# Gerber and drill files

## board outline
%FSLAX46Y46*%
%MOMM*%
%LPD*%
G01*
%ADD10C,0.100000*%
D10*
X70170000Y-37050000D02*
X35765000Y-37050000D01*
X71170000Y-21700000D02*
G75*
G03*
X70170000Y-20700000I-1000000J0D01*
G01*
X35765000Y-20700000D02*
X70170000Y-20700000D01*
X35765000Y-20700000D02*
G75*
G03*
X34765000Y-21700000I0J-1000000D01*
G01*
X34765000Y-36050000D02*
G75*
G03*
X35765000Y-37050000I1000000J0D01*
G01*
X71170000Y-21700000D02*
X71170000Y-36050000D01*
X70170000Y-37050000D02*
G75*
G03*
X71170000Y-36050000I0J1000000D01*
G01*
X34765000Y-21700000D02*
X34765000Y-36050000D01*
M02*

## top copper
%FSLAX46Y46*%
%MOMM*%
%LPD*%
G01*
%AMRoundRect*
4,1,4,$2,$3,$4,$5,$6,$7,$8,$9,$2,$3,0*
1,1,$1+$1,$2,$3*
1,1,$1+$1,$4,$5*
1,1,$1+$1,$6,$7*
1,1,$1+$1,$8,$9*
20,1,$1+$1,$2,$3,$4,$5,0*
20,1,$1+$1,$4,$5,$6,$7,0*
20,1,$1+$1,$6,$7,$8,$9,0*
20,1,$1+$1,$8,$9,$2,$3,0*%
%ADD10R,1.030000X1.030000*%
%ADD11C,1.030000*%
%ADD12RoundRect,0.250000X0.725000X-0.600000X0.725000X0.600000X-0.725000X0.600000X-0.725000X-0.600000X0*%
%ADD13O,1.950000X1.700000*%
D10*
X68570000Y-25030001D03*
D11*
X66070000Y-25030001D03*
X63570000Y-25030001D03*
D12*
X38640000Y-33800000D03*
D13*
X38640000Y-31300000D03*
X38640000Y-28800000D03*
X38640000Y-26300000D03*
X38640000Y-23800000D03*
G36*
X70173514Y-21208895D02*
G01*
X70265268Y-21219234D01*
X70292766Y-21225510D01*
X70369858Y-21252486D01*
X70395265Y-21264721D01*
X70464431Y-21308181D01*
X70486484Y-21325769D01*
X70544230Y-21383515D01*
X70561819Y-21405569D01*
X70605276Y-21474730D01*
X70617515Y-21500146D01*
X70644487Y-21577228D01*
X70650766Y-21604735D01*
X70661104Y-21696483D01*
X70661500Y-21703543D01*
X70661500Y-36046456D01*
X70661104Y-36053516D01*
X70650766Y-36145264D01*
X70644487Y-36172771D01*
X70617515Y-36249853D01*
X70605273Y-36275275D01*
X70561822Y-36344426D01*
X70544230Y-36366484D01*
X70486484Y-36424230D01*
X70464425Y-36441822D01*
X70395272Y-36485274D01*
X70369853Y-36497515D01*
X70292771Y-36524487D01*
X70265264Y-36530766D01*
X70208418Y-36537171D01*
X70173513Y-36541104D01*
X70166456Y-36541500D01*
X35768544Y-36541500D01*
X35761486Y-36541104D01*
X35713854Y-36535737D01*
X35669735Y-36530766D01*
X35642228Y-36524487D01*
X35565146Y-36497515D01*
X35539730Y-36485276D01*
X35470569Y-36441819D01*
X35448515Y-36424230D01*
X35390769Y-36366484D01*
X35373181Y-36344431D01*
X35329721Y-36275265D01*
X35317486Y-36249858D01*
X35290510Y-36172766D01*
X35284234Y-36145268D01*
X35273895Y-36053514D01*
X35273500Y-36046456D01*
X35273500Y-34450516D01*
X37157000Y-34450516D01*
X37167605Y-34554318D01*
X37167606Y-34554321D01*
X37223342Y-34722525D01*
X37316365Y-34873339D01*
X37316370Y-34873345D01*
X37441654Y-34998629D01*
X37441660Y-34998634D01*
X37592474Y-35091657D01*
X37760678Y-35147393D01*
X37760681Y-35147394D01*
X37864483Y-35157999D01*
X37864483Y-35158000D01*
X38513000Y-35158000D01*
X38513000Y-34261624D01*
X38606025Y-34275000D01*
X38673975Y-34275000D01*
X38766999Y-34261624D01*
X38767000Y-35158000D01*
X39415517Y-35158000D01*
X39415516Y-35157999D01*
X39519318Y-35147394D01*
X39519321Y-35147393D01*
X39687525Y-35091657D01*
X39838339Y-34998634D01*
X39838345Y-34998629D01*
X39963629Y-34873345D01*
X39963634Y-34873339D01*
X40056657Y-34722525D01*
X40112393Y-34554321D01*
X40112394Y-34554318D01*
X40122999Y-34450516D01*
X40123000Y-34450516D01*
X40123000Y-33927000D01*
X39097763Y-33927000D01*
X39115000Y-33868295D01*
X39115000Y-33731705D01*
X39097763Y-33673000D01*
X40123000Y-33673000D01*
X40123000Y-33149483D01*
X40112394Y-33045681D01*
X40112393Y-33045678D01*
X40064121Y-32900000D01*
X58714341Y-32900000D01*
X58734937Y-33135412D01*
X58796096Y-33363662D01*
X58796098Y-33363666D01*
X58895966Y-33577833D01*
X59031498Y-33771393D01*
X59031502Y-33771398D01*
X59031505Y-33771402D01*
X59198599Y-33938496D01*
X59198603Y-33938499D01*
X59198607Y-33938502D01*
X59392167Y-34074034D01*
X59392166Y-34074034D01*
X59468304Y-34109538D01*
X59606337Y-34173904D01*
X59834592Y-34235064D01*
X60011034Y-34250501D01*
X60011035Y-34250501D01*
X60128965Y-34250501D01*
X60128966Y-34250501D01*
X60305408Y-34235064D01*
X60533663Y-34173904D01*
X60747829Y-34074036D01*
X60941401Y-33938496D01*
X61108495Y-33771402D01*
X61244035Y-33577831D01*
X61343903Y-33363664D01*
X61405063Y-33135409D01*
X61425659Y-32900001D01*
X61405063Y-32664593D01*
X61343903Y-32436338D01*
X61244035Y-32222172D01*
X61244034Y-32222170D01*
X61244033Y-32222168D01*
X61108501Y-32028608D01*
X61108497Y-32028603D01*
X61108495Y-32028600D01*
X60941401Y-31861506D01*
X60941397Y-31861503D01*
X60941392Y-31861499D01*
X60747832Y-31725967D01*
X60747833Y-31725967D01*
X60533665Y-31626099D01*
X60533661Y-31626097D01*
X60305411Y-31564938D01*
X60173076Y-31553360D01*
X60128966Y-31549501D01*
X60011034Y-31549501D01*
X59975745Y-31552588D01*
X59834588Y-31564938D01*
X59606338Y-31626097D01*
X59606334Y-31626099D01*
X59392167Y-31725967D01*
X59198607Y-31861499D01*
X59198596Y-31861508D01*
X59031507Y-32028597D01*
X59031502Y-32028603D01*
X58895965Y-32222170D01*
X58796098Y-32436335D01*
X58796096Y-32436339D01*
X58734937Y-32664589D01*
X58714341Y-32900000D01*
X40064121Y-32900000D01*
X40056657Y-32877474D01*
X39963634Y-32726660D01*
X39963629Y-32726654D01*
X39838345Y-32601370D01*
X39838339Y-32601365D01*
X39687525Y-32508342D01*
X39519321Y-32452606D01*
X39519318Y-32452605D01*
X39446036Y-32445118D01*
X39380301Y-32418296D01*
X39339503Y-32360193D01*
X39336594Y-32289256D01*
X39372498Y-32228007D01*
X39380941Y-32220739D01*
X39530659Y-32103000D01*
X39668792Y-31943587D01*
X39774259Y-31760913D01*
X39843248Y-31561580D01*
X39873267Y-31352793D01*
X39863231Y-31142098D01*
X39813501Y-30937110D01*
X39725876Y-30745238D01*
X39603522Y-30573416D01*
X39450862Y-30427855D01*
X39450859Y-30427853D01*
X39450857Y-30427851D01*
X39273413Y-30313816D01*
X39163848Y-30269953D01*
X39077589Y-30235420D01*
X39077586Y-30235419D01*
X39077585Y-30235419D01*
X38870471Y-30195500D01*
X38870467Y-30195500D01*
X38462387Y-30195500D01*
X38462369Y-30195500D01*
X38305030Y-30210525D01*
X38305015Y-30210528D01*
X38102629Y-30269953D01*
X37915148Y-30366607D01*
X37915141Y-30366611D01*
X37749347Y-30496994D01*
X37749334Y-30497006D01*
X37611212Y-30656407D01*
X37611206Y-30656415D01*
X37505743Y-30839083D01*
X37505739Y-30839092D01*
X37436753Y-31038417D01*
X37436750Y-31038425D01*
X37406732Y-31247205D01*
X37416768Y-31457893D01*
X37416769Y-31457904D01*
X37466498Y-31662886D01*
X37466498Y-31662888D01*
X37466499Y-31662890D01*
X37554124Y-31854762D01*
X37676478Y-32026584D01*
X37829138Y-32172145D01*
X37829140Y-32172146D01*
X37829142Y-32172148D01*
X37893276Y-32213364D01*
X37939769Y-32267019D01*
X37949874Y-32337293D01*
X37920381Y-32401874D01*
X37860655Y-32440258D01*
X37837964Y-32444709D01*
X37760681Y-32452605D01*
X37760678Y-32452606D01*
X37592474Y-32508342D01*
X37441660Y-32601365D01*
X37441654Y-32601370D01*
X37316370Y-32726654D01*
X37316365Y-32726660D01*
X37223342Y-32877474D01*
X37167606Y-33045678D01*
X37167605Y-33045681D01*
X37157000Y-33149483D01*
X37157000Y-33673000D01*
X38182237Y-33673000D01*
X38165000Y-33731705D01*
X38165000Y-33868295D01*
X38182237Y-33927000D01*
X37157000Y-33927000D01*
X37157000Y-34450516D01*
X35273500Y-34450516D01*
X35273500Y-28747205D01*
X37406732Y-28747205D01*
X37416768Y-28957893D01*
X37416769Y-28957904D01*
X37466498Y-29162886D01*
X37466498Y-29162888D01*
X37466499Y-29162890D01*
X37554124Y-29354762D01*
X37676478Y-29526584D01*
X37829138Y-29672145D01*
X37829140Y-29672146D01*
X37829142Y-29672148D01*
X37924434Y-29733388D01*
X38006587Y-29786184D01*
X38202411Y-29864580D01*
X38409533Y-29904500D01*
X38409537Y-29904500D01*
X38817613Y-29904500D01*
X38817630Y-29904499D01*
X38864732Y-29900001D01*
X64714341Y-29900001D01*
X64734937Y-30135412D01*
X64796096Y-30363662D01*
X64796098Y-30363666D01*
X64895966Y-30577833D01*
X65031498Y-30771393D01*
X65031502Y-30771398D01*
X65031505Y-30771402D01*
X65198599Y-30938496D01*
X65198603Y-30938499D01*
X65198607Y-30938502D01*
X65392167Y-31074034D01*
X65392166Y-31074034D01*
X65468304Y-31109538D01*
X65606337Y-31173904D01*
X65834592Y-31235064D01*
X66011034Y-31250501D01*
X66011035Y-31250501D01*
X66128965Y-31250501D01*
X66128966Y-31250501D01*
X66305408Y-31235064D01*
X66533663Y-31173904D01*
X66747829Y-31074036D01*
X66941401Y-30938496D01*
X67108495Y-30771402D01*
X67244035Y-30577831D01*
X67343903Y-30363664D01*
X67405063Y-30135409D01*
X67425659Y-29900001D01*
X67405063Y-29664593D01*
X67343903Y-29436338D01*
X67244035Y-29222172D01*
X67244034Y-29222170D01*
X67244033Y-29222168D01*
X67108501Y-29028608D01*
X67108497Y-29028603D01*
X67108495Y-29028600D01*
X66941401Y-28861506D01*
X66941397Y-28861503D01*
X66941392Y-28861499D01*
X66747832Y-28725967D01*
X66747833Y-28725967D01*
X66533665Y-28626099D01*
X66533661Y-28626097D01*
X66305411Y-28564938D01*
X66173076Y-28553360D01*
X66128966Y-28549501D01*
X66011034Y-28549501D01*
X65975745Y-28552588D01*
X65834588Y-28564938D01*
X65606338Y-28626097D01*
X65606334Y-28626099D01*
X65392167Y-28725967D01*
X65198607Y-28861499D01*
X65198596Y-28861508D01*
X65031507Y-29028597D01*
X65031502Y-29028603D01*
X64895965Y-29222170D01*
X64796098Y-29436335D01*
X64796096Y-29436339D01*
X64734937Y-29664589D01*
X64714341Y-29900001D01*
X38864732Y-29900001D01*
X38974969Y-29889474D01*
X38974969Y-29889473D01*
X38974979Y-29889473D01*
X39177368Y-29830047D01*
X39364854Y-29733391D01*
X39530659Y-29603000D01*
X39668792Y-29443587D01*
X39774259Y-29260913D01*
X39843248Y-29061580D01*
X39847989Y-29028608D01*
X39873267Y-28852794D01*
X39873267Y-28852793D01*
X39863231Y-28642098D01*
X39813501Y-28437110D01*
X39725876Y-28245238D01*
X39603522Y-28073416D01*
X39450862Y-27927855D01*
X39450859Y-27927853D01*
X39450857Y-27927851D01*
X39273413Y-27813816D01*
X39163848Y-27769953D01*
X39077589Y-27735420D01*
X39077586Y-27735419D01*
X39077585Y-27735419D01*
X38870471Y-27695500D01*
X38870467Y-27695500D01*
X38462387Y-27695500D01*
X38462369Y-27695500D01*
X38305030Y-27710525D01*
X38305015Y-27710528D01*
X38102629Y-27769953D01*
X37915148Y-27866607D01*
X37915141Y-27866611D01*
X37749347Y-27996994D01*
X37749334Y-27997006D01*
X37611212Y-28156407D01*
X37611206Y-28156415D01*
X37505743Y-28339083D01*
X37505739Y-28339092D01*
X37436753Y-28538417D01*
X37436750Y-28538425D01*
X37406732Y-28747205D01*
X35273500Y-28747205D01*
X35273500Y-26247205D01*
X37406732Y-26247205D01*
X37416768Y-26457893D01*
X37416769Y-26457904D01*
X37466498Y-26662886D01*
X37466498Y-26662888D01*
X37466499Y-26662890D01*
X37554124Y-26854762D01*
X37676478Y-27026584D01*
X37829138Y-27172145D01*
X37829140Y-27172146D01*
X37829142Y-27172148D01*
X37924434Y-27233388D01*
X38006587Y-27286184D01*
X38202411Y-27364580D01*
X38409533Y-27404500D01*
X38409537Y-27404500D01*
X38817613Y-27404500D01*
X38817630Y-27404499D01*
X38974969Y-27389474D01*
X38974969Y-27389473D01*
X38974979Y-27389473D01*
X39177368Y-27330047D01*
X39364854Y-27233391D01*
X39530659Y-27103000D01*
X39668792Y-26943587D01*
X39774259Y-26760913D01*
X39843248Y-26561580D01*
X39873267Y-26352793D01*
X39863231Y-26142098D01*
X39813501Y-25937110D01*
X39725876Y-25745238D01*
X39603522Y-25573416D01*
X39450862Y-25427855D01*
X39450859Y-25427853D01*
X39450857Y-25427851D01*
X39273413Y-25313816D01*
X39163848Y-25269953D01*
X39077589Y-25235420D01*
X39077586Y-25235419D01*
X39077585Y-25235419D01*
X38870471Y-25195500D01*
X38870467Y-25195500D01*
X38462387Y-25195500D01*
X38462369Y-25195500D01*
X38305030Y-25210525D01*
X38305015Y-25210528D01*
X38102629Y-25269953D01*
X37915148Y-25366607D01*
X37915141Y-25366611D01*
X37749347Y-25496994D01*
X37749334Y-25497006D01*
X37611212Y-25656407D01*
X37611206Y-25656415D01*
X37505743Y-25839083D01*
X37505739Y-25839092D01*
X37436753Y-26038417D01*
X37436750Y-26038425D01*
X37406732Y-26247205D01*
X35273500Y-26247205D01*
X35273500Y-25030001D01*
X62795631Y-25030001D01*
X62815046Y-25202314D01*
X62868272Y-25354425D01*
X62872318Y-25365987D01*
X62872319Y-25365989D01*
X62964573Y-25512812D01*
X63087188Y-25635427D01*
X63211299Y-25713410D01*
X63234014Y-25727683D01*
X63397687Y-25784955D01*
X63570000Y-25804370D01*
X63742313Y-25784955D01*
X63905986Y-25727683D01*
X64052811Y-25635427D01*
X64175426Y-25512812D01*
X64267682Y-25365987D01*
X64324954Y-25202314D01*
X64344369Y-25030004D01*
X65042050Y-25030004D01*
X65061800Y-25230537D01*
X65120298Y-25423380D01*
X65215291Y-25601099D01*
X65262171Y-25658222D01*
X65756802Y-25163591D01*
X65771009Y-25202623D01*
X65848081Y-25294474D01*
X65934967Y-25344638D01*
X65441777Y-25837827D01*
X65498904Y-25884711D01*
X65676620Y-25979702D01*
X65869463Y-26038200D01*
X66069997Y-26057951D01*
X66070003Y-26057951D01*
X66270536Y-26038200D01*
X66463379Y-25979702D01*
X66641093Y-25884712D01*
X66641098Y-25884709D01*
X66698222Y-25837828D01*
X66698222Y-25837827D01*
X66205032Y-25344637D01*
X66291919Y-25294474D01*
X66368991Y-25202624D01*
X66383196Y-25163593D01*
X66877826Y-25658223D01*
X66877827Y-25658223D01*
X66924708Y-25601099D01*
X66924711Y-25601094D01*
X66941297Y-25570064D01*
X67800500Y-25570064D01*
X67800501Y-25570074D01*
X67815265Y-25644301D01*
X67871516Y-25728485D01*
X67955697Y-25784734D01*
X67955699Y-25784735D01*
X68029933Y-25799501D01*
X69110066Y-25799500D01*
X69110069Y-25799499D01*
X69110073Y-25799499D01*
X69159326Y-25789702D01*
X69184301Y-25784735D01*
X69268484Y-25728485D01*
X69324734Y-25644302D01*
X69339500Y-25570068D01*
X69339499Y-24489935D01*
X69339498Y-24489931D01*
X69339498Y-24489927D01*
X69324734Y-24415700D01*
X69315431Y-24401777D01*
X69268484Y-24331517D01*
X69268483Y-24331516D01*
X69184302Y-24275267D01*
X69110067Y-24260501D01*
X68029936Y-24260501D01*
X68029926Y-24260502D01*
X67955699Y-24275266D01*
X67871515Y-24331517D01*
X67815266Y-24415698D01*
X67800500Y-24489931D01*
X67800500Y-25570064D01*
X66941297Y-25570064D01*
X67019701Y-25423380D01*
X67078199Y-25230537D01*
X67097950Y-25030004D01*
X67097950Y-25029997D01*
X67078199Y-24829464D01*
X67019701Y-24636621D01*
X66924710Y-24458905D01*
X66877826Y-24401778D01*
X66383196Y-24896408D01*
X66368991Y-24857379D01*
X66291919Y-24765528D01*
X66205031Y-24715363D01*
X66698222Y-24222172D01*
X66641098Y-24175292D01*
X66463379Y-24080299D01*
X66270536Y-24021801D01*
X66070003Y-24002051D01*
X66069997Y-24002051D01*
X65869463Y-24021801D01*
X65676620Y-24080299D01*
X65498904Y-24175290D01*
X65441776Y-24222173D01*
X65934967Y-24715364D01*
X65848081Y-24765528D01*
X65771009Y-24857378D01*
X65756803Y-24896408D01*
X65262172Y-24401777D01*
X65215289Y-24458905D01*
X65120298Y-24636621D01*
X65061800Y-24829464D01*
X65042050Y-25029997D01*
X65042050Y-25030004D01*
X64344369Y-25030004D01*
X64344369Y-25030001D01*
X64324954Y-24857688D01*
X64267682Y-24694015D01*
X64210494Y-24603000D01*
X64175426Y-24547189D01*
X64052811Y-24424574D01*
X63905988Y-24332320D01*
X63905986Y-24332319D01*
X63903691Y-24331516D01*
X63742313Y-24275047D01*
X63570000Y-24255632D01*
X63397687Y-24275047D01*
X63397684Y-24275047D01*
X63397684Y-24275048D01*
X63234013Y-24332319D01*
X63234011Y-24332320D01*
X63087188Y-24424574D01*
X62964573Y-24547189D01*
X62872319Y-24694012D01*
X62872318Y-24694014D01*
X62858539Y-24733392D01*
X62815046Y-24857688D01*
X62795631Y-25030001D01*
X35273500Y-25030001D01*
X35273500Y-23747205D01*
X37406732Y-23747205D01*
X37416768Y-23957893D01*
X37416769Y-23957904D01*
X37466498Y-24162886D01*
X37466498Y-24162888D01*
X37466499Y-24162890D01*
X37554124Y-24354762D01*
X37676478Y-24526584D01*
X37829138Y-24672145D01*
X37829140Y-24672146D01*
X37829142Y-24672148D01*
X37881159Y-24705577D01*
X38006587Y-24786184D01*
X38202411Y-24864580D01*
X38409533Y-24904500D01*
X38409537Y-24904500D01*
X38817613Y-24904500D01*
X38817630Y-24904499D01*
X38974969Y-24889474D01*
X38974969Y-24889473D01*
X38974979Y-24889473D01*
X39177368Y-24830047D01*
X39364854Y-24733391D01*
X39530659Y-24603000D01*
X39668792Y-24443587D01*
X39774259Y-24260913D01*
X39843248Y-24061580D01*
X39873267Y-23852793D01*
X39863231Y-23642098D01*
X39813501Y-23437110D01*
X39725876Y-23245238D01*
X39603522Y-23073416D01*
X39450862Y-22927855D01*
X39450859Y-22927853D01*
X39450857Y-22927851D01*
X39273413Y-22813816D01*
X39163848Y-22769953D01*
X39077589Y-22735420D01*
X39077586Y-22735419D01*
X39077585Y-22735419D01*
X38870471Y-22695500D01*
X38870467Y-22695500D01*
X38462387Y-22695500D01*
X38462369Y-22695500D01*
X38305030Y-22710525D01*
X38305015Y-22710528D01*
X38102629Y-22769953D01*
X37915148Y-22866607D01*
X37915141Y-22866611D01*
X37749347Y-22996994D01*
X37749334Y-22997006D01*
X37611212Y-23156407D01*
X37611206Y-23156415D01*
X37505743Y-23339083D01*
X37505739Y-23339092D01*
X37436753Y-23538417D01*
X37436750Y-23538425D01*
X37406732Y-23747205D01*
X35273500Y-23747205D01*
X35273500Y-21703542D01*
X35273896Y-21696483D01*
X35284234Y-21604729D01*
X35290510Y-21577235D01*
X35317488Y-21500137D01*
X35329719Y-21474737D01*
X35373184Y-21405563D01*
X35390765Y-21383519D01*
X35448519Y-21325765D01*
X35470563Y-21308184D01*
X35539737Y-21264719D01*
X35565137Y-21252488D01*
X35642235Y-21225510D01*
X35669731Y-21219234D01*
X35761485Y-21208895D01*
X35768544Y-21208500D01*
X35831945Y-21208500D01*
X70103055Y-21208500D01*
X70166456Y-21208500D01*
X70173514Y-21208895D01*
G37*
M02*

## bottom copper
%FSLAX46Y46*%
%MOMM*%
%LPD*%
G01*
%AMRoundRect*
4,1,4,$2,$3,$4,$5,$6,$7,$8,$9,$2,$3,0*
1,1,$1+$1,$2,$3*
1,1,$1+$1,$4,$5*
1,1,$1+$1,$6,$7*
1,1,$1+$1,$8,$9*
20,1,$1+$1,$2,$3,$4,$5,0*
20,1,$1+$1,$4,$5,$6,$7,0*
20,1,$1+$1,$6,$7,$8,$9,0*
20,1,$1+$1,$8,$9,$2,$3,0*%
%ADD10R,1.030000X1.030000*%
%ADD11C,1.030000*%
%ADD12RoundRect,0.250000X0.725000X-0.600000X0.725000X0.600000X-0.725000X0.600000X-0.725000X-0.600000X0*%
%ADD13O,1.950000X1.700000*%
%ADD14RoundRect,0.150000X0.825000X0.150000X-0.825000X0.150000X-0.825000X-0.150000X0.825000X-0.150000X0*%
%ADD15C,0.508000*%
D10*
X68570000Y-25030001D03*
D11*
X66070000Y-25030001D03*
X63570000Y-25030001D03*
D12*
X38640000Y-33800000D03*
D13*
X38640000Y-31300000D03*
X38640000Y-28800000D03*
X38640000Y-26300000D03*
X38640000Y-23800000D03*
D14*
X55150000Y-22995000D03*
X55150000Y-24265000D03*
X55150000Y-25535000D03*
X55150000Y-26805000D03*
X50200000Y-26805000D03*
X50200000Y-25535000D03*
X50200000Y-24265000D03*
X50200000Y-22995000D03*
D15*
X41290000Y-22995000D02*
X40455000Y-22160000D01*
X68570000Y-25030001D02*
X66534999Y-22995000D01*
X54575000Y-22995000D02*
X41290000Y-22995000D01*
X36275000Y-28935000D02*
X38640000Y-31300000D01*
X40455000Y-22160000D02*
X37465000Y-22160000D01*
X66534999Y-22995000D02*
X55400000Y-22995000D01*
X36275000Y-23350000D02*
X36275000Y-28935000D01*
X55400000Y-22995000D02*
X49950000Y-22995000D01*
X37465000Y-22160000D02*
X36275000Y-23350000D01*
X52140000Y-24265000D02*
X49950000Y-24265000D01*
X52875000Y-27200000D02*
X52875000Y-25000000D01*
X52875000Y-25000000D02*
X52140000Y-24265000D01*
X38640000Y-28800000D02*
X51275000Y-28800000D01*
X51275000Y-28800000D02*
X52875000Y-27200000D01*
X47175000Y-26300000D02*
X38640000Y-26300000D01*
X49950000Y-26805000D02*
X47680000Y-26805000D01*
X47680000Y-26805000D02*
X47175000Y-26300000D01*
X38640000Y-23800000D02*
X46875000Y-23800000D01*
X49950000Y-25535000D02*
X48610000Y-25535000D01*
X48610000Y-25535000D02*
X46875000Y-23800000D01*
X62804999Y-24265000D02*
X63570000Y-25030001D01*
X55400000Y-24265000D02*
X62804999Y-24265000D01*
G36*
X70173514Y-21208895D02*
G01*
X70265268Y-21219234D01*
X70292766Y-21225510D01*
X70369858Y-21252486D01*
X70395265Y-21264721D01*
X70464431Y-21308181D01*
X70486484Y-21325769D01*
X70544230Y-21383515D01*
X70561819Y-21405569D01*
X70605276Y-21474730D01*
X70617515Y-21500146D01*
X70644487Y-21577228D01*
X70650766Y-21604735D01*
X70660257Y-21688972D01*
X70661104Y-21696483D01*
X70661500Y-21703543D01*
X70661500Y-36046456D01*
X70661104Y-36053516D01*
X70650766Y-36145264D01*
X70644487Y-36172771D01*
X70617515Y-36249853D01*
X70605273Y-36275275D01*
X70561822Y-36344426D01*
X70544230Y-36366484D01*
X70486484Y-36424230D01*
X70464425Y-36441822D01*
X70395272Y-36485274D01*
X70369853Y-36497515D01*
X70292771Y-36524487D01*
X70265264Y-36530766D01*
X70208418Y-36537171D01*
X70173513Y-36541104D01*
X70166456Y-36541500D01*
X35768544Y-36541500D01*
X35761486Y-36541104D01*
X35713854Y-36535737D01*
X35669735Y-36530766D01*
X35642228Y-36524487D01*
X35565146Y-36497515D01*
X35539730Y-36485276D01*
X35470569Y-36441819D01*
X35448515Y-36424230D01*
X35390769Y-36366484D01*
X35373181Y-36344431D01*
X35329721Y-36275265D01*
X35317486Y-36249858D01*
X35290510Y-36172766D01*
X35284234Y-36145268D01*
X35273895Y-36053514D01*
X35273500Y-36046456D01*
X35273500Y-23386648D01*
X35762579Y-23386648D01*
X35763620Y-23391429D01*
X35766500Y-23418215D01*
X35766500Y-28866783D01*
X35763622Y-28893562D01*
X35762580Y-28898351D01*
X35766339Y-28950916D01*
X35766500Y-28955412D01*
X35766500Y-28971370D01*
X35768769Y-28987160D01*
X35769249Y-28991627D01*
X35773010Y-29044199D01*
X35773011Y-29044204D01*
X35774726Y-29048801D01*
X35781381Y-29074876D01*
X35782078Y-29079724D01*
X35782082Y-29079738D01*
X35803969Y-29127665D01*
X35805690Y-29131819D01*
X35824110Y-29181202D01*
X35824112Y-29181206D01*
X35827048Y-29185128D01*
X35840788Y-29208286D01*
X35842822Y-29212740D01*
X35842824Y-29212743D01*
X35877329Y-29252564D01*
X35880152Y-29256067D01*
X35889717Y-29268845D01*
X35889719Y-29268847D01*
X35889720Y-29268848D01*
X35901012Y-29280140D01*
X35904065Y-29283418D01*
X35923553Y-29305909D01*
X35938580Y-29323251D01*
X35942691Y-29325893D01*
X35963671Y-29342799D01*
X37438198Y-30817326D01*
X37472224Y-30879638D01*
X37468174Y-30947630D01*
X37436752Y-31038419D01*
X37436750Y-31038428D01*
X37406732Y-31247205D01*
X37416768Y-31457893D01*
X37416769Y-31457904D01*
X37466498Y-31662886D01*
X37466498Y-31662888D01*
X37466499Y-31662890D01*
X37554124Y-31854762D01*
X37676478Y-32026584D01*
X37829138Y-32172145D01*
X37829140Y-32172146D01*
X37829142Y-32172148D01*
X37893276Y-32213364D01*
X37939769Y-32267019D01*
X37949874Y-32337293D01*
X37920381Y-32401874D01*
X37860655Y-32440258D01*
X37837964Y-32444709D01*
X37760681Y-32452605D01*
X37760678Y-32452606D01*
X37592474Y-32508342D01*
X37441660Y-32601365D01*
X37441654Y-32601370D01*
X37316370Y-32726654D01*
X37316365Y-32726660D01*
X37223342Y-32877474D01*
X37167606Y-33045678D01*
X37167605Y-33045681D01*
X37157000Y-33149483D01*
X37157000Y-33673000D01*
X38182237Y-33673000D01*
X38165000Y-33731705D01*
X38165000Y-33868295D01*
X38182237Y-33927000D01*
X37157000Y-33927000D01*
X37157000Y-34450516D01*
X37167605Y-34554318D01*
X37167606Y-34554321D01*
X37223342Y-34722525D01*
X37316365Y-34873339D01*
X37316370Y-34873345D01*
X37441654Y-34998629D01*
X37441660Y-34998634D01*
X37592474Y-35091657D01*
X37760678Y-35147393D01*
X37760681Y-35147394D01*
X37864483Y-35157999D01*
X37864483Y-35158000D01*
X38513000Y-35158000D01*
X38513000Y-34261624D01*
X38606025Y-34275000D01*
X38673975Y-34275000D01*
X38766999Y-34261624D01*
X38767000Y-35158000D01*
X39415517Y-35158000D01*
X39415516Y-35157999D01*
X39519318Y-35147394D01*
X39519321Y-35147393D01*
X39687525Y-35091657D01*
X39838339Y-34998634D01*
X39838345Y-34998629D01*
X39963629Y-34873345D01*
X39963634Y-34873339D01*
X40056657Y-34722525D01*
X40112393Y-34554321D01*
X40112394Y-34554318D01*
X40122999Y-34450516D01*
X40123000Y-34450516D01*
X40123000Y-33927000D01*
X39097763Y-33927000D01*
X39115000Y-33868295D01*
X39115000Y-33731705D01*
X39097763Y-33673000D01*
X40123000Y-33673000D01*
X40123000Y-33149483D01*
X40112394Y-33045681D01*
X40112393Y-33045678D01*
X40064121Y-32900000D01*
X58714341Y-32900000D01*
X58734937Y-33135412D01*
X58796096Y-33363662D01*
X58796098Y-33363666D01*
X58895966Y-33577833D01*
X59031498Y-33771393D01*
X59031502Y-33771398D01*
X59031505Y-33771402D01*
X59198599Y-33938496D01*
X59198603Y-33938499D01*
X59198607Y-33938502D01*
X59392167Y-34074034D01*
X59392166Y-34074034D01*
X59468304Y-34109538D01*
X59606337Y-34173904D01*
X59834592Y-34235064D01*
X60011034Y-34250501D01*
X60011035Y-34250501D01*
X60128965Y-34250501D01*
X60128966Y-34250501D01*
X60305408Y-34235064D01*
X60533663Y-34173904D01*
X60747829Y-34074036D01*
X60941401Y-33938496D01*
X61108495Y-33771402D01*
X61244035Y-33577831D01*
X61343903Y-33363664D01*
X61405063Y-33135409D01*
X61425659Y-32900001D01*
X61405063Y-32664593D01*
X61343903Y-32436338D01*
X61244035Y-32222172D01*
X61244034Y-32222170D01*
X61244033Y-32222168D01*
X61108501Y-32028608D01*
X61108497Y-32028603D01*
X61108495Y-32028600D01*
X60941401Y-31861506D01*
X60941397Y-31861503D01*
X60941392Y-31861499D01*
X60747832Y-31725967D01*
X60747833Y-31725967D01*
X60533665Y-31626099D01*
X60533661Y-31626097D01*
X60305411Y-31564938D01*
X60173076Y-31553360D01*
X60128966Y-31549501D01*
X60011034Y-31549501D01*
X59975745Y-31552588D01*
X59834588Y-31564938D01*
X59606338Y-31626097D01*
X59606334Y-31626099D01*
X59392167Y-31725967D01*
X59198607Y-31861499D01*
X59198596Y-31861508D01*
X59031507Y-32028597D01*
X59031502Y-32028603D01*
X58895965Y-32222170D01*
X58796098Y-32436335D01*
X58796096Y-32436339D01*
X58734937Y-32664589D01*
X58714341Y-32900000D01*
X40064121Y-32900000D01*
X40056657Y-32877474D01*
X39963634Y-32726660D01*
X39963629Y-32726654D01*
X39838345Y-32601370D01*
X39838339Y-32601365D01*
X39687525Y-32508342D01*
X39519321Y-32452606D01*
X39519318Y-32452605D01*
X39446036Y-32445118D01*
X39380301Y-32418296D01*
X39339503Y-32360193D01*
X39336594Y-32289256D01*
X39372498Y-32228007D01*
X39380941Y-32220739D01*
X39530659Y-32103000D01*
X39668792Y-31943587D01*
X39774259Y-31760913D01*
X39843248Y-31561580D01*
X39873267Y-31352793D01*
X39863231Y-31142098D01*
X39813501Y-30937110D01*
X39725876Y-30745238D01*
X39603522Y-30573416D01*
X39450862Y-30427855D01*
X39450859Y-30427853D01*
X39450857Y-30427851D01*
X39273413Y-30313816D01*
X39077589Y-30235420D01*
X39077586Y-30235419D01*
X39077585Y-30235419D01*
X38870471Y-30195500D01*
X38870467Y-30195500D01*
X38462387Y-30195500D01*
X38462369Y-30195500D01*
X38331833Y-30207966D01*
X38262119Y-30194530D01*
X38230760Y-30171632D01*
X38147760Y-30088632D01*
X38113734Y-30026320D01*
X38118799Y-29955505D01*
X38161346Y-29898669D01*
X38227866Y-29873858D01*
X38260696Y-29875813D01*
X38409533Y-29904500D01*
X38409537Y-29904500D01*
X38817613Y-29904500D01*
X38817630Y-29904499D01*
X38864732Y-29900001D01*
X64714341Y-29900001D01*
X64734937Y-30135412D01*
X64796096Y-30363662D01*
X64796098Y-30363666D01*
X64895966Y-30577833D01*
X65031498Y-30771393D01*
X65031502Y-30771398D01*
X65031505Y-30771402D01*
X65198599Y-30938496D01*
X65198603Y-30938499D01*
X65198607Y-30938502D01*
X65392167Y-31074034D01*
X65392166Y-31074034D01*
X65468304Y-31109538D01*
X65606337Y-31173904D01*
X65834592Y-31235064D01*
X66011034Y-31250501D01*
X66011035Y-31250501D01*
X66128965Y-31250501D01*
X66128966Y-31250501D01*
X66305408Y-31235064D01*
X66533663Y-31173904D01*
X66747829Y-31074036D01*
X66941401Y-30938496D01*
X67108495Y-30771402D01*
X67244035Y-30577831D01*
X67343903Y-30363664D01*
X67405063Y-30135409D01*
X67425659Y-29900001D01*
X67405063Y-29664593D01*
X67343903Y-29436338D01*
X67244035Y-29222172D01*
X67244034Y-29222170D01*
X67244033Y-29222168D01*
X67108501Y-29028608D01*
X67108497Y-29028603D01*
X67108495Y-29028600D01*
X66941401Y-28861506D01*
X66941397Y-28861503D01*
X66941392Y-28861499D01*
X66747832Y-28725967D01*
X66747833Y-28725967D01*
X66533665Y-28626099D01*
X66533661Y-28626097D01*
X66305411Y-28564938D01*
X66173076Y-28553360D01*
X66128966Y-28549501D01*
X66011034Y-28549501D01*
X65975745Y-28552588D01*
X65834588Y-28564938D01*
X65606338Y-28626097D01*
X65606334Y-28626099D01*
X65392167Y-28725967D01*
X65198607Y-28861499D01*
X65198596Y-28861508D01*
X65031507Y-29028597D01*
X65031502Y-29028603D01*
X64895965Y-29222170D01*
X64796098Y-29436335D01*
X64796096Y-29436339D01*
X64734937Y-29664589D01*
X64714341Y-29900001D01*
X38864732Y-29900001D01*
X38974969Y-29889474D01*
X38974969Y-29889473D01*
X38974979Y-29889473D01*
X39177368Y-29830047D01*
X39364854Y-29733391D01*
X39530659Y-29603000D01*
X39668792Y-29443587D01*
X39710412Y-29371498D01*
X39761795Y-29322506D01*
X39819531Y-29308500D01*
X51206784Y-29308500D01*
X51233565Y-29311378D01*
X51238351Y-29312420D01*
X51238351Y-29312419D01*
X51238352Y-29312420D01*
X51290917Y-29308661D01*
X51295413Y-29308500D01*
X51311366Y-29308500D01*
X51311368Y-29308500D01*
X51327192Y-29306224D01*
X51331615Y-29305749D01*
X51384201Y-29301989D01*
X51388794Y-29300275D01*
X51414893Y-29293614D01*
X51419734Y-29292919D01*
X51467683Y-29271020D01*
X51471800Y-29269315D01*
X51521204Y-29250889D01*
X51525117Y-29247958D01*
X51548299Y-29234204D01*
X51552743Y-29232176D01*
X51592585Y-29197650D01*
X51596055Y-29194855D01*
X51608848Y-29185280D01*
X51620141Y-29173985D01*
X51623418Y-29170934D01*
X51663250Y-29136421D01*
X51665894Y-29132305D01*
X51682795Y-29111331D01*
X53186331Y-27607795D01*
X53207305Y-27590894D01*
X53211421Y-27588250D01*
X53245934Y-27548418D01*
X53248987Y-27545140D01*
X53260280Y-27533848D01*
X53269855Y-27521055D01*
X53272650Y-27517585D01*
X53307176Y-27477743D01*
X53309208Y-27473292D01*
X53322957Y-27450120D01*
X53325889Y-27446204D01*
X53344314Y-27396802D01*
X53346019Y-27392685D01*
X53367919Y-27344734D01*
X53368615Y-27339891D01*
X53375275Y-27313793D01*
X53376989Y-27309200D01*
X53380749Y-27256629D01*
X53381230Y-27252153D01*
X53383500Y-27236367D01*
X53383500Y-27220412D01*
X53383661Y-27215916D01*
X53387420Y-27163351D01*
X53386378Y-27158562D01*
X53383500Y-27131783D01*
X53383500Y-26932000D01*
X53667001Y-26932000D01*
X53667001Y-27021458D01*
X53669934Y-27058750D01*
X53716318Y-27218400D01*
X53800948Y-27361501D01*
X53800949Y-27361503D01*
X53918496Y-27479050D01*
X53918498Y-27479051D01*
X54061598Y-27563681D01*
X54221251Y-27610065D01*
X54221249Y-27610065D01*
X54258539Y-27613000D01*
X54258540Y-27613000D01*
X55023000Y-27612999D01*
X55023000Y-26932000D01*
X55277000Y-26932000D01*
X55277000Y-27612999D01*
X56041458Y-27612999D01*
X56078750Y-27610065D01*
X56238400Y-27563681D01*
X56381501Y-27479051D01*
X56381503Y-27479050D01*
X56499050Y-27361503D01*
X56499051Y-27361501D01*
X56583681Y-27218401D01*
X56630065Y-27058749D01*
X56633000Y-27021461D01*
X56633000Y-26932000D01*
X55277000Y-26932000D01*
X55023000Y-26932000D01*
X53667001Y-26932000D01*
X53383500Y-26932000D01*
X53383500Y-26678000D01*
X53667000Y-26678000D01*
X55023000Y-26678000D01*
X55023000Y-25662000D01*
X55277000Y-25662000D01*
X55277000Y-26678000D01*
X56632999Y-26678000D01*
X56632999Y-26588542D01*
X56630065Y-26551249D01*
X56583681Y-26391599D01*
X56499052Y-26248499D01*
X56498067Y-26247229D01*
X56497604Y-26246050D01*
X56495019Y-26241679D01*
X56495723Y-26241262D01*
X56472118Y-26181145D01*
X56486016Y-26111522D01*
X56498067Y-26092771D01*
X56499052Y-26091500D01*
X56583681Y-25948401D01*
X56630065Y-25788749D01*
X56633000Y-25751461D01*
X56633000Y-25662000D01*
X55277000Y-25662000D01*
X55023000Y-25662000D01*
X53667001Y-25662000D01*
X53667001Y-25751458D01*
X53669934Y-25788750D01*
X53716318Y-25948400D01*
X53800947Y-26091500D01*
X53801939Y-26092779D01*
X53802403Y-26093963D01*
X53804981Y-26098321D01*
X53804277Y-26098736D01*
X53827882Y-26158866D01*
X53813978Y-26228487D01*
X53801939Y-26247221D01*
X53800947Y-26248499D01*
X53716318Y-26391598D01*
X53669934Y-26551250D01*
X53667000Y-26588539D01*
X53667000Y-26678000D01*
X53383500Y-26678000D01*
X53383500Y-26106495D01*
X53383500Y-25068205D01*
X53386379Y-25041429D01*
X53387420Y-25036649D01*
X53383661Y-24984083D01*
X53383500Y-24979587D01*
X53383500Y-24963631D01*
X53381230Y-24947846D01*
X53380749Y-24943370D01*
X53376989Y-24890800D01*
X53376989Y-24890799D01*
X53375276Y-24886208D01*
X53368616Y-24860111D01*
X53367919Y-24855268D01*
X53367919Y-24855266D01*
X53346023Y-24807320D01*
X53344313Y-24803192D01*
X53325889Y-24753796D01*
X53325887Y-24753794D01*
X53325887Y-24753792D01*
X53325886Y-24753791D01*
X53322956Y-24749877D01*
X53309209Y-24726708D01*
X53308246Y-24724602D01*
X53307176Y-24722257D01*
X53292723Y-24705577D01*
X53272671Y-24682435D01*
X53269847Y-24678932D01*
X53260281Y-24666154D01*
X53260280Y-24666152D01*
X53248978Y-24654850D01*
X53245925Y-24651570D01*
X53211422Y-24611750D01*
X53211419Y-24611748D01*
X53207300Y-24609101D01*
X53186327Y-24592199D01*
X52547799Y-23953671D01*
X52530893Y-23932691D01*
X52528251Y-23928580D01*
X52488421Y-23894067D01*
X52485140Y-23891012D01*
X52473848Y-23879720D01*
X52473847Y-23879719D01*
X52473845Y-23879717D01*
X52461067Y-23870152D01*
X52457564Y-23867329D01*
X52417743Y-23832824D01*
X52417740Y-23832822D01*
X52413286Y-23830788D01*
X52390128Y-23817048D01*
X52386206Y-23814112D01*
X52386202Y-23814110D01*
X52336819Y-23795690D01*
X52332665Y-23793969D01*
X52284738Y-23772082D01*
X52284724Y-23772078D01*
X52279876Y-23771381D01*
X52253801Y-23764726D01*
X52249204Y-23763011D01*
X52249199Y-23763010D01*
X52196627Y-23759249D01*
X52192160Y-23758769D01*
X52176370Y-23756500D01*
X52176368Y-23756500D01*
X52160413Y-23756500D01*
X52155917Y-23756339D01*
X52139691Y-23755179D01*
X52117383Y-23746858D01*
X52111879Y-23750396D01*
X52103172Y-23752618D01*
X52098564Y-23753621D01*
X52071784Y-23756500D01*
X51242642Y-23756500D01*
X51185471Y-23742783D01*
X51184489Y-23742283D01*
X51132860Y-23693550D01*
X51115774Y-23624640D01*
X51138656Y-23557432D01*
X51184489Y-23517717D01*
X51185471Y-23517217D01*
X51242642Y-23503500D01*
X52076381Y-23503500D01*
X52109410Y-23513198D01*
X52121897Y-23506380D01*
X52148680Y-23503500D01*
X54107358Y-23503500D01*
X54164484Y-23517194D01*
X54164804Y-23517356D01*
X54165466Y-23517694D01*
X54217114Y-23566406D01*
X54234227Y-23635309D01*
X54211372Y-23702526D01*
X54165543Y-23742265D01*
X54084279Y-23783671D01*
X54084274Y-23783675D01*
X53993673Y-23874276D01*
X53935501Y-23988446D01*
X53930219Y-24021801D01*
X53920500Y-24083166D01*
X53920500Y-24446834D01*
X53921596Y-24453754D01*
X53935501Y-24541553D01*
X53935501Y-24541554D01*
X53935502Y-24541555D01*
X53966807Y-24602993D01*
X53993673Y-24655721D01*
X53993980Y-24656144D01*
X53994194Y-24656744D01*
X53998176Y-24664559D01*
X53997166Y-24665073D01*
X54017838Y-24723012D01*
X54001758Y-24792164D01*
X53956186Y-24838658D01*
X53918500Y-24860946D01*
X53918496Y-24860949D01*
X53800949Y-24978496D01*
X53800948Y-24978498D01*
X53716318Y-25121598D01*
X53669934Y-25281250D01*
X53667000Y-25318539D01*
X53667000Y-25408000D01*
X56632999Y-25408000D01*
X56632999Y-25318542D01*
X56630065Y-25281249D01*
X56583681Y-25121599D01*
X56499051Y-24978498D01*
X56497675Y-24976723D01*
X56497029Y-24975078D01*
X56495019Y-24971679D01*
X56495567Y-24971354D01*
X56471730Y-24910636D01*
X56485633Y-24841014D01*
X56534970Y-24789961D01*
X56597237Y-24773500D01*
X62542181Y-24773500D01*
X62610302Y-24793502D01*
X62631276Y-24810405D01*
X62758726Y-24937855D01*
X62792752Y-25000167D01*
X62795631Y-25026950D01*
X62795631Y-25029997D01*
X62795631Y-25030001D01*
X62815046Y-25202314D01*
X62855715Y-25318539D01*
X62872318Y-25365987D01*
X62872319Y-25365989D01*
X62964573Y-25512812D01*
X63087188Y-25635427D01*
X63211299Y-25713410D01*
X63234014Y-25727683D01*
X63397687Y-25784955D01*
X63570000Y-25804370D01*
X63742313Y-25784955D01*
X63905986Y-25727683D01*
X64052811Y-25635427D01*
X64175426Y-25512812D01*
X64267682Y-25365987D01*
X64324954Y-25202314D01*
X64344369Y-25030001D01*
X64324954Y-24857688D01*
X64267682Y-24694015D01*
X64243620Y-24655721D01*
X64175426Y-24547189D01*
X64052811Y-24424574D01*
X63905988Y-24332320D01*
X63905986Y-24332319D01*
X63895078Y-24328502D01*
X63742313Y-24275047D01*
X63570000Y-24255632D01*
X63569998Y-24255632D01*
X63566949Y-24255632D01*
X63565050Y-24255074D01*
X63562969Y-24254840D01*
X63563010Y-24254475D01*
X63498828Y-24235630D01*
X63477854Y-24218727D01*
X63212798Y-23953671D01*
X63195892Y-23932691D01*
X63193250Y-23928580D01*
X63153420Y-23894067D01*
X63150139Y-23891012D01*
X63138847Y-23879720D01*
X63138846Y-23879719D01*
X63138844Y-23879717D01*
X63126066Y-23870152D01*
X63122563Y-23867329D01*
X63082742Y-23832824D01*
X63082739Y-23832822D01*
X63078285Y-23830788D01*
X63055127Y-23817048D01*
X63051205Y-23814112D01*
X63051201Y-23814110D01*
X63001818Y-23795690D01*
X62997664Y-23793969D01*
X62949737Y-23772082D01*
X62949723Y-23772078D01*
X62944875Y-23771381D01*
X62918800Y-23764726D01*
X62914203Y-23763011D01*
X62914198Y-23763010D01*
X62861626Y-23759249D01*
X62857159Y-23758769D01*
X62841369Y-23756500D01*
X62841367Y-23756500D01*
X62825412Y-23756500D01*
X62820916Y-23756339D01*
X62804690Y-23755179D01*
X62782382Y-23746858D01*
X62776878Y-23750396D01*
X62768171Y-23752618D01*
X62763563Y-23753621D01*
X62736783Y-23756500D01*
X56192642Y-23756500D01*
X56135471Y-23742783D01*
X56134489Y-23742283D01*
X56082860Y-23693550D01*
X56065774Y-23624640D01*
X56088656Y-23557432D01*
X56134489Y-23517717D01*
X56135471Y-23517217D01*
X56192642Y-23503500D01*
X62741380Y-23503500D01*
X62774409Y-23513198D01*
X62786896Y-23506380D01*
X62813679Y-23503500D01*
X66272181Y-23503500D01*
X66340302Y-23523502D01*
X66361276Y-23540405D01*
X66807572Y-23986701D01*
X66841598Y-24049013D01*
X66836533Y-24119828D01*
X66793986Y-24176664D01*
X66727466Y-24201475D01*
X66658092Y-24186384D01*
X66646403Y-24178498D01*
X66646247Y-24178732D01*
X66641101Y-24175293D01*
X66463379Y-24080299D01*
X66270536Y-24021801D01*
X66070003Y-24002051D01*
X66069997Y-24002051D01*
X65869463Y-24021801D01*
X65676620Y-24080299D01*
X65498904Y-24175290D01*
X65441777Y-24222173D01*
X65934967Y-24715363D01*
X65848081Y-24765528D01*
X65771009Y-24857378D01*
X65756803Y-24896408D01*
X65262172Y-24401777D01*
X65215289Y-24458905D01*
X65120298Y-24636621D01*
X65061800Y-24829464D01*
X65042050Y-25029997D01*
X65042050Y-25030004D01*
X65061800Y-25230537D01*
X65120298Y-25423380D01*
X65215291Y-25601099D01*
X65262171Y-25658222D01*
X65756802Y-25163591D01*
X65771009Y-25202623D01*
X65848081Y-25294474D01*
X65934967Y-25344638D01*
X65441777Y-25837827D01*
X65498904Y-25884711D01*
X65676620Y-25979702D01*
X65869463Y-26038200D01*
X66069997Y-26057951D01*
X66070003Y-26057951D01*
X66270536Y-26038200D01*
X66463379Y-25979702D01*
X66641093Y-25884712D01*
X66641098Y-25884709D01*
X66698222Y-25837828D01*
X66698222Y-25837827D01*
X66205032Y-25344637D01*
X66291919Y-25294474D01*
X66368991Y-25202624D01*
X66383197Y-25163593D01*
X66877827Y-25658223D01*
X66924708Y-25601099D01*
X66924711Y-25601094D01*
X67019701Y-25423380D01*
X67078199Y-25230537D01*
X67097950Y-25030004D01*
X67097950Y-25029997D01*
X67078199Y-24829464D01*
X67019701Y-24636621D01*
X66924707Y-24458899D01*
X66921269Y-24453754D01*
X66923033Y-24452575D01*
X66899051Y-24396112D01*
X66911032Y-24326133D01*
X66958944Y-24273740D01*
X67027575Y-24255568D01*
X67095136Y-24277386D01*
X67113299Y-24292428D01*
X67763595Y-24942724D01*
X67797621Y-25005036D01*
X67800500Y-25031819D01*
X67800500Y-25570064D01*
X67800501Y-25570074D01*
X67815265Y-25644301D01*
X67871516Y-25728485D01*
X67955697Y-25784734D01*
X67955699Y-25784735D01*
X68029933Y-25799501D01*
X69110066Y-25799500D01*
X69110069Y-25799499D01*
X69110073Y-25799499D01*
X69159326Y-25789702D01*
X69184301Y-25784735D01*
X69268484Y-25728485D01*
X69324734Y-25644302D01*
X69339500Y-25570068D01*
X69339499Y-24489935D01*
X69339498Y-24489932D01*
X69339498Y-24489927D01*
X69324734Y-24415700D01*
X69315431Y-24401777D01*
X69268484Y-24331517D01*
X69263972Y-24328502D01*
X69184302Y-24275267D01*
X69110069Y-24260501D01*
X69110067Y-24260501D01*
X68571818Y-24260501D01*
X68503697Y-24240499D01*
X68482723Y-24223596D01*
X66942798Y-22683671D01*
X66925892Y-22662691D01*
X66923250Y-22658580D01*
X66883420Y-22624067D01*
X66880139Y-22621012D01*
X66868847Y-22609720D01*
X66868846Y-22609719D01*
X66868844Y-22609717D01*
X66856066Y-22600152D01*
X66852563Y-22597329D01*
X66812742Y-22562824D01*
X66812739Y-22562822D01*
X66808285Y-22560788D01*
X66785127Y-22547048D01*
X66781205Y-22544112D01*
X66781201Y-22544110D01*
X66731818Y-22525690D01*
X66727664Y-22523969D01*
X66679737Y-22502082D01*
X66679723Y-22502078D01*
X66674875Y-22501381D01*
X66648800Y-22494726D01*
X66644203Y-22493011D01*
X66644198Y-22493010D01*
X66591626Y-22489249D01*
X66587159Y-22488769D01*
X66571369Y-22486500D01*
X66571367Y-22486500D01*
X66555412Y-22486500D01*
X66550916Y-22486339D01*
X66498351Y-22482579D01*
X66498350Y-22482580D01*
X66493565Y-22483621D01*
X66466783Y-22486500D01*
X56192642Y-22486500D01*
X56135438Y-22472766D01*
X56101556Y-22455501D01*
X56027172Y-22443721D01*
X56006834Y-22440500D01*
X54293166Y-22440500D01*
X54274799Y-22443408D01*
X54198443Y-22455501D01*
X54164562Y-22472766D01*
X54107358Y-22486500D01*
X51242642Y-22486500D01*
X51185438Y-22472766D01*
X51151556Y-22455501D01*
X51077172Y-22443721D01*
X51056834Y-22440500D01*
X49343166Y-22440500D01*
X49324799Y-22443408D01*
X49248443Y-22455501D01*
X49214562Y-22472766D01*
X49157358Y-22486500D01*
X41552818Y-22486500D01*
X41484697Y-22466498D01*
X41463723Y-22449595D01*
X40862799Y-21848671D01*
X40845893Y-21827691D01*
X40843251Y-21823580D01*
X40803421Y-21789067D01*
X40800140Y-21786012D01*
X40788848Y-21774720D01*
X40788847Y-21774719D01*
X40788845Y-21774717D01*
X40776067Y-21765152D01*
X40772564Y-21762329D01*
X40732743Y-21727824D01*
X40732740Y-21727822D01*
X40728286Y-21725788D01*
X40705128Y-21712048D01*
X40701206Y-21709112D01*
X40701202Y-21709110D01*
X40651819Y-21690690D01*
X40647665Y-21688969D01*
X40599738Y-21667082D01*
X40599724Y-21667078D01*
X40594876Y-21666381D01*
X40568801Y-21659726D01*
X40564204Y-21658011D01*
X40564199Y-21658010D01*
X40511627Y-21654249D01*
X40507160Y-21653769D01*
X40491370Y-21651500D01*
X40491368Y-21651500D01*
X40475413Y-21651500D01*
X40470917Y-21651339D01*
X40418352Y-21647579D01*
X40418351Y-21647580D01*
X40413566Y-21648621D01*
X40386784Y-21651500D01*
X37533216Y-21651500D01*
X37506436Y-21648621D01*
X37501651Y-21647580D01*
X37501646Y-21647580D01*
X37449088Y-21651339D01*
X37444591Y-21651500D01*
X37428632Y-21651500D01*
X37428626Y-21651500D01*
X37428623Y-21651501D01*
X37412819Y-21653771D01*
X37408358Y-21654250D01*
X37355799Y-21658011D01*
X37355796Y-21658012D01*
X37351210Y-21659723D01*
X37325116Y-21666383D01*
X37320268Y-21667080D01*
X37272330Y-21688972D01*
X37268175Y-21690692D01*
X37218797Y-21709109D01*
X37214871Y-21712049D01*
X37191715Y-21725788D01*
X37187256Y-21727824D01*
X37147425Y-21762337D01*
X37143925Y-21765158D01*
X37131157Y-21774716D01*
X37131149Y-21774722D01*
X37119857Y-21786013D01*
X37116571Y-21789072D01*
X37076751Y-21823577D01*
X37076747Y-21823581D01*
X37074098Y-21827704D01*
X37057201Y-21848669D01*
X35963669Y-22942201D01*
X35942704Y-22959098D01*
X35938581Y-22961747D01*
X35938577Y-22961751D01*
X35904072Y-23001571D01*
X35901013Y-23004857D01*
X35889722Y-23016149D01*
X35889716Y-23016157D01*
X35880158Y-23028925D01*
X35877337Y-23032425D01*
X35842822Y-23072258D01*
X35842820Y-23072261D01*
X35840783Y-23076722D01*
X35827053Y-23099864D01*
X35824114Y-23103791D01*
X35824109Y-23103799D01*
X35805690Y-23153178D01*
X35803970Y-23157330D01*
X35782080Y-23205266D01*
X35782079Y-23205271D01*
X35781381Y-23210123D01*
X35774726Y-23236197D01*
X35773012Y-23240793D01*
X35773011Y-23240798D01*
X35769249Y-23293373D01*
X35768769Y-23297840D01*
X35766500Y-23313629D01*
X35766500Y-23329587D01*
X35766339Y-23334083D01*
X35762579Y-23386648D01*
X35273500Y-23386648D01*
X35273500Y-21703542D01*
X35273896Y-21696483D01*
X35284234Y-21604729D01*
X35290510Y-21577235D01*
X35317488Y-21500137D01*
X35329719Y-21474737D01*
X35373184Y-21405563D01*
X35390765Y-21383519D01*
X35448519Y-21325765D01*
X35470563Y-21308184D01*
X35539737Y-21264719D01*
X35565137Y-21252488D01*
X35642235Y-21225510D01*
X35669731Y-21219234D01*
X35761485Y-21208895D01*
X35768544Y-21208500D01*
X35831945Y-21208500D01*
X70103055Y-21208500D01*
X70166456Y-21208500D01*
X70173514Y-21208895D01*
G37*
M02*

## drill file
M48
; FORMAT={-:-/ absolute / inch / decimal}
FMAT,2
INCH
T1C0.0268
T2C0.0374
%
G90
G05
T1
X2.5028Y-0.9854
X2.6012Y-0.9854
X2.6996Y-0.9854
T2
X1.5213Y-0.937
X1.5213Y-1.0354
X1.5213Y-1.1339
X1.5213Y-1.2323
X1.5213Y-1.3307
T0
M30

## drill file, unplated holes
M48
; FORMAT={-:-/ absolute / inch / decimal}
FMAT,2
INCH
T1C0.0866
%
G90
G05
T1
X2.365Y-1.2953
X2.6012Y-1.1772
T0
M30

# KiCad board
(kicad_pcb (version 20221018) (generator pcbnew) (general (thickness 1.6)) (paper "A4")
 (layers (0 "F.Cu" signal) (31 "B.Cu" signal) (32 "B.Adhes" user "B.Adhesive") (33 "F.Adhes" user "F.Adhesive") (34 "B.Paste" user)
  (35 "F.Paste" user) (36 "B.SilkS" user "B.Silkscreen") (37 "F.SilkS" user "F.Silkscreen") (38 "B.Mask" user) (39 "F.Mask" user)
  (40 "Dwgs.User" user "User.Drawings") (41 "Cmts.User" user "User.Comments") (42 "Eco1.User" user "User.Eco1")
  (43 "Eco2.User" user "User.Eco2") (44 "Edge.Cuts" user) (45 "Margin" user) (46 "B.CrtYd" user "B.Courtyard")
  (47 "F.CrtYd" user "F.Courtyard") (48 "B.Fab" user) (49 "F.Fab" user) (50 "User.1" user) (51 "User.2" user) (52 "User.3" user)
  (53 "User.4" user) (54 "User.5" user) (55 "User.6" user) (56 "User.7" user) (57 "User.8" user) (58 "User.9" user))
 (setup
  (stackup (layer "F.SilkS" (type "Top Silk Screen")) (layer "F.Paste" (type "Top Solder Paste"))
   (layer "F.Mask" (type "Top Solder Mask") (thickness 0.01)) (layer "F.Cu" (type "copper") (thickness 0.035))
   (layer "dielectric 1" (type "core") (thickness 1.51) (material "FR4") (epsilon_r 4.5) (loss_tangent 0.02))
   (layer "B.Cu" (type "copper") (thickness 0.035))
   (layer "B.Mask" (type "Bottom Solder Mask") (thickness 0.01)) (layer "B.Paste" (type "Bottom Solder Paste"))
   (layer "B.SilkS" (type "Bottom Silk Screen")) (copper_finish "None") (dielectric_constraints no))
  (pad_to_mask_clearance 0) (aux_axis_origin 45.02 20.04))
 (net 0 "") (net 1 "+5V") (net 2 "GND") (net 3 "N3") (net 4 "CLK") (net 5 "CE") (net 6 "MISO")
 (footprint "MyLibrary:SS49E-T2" (layer "F.Cu") (at 66.07 25.030001 180)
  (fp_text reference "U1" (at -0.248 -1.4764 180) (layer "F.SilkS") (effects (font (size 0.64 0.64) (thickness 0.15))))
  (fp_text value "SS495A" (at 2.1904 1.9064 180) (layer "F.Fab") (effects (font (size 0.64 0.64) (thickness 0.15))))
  (pad "1" thru_hole rect (at -2.5 0 180) (size 1.03 1.03) (drill 0.68) (layers "*.Cu" "*.Mask") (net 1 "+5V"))
  (pad "2" thru_hole circle (at 0 0 180) (size 1.03 1.03) (drill 0.68) (layers "*.Cu" "*.Mask") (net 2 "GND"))
  (pad "3" thru_hole circle (at 2.5 0 180) (size 1.03 1.03) (drill 0.68) (layers "*.Cu" "*.Mask") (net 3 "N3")))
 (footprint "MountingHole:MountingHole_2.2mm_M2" (layer "F.Cu") (at 60.07 32.900001)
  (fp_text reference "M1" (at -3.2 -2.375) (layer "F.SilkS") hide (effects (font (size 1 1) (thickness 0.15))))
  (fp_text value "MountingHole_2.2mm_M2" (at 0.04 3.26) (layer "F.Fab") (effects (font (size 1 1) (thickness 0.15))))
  (pad "" np_thru_hole circle (at 0 0) (size 2.2 2.2) (drill 2.2) (layers "*.Cu" "*.Mask")))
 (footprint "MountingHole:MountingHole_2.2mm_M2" (layer "F.Cu") (at 66.07 29.900001)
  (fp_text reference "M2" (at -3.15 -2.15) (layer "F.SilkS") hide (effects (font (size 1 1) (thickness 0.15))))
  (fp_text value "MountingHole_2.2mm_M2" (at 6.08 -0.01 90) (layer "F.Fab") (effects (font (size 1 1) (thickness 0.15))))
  (pad "" np_thru_hole circle (at 0 0) (size 2.2 2.2) (drill 2.2) (layers "*.Cu" "*.Mask")))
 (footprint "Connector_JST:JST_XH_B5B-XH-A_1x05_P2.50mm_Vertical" (layer "F.Cu") (at 38.64 33.8 90)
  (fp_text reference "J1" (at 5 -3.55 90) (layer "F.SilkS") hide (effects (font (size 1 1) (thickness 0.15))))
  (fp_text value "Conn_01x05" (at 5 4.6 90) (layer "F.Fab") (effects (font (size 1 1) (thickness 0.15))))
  (pad "1" thru_hole roundrect (at 0 0 90) (size 1.7 1.95) (drill 0.95) (layers "*.Cu" "*.Mask") (roundrect_rratio 0.1470588235)
   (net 2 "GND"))
  (pad "2" thru_hole oval (at 2.5 0 90) (size 1.7 1.95) (drill 0.95) (layers "*.Cu" "*.Mask") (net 1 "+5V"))
  (pad "3" thru_hole oval (at 5 0 90) (size 1.7 1.95) (drill 0.95) (layers "*.Cu" "*.Mask") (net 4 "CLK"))
  (pad "4" thru_hole oval (at 7.5 0 90) (size 1.7 1.95) (drill 0.95) (layers "*.Cu" "*.Mask") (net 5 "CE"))
  (pad "5" thru_hole oval (at 10 0 90) (size 1.7 1.95) (drill 0.95) (layers "*.Cu" "*.Mask") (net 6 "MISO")))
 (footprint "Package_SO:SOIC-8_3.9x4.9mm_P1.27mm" (layer "B.Cu") (at 52.675 24.9 180)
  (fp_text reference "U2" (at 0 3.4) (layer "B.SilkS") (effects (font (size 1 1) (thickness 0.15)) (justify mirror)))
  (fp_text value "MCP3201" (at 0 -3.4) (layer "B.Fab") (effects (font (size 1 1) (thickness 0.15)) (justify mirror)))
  (pad "1" smd roundrect (at -2.475 1.905 180) (size 1.95 0.6) (layers "B.Cu" "B.Paste" "B.Mask") (roundrect_rratio 0.25) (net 1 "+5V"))
  (pad "2" smd roundrect (at -2.475 0.635 180) (size 1.95 0.6) (layers "B.Cu" "B.Paste" "B.Mask") (roundrect_rratio 0.25) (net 3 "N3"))
  (pad "3" smd roundrect (at -2.475 -0.635 180) (size 1.95 0.6) (layers "B.Cu" "B.Paste" "B.Mask") (roundrect_rratio 0.25) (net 2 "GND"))
  (pad "4" smd roundrect (at -2.475 -1.905 180) (size 1.95 0.6) (layers "B.Cu" "B.Paste" "B.Mask") (roundrect_rratio 0.25) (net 2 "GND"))
  (pad "5" smd roundrect (at 2.475 -1.905 180) (size 1.95 0.6) (layers "B.Cu" "B.Paste" "B.Mask") (roundrect_rratio 0.25) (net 5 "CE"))
  (pad "6" smd roundrect (at 2.475 -0.635 180) (size 1.95 0.6) (layers "B.Cu" "B.Paste" "B.Mask") (roundrect_rratio 0.25) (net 6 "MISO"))
  (pad "7" smd roundrect (at 2.475 0.635 180) (size 1.95 0.6) (layers "B.Cu" "B.Paste" "B.Mask") (roundrect_rratio 0.25) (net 4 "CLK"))
  (pad "8" smd roundrect (at 2.475 1.905 180) (size 1.95 0.6) (layers "B.Cu" "B.Paste" "B.Mask") (roundrect_rratio 0.25) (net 1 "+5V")))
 (gr_line (start 70.17 37.05) (end 35.765 37.05) (stroke (width 0.1) (type solid)) (layer "Edge.Cuts"))
 (gr_arc (start 70.17 20.7) (mid 70.877107 20.992893) (end 71.17 21.7) (stroke (width 0.1) (type solid)) (layer "Edge.Cuts"))
 (gr_line (start 35.765 20.7) (end 70.17 20.7) (stroke (width 0.1) (type solid)) (layer "Edge.Cuts"))
 (gr_arc (start 34.765 21.7) (mid 35.057893 20.992893) (end 35.765 20.7) (stroke (width 0.1) (type solid)) (layer "Edge.Cuts"))
 (gr_arc (start 35.765 37.05) (mid 35.057893 36.757107) (end 34.765 36.05) (stroke (width 0.1) (type solid)) (layer "Edge.Cuts"))
 (gr_line (start 71.17 21.7) (end 71.17 36.05) (stroke (width 0.1) (type solid)) (layer "Edge.Cuts"))
 (gr_arc (start 71.17 36.05) (mid 70.877107 36.757107) (end 70.17 37.05) (stroke (width 0.1) (type solid)) (layer "Edge.Cuts"))
 (gr_line (start 34.765 21.7) (end 34.765 36.05) (stroke (width 0.1) (type solid)) (layer "Edge.Cuts"))
 (segment (start 41.29 22.995) (end 40.455 22.16) (width 0.508) (layer "B.Cu") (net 1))
 (segment (start 68.57 25.030001) (end 66.534999 22.995) (width 0.508) (layer "B.Cu") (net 1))
 (segment (start 54.575 22.995) (end 41.29 22.995) (width 0.508) (layer "B.Cu") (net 1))
 (segment (start 36.275 28.935) (end 38.64 31.3) (width 0.508) (layer "B.Cu") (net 1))
 (segment (start 40.455 22.16) (end 37.465 22.16) (width 0.508) (layer "B.Cu") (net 1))
 (segment (start 66.534999 22.995) (end 55.4 22.995) (width 0.508) (layer "B.Cu") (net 1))
 (segment (start 36.275 23.35) (end 36.275 28.935) (width 0.508) (layer "B.Cu") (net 1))
 (segment (start 55.4 22.995) (end 49.95 22.995) (width 0.508) (layer "B.Cu") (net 1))
 (segment (start 37.465 22.16) (end 36.275 23.35) (width 0.508) (layer "B.Cu") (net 1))
 (segment (start 52.14 24.265) (end 49.95 24.265) (width 0.508) (layer "B.Cu") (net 4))
 (segment (start 52.875 27.2) (end 52.875 25) (width 0.508) (layer "B.Cu") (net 4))
 (segment (start 52.875 25) (end 52.14 24.265) (width 0.508) (layer "B.Cu") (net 4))
 (segment (start 38.64 28.8) (end 51.275 28.8) (width 0.508) (layer "B.Cu") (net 4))
 (segment (start 51.275 28.8) (end 52.875 27.2) (width 0.508) (layer "B.Cu") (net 4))
 (segment (start 47.175 26.3) (end 38.64 26.3) (width 0.508) (layer "B.Cu") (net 5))
 (segment (start 49.95 26.805) (end 47.68 26.805) (width 0.508) (layer "B.Cu") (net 5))
 (segment (start 47.68 26.805) (end 47.175 26.3) (width 0.508) (layer "B.Cu") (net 5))
 (segment (start 38.64 23.8) (end 46.875 23.8) (width 0.508) (layer "B.Cu") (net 6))
 (segment (start 49.95 25.535) (end 48.61 25.535) (width 0.508) (layer "B.Cu") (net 6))
 (segment (start 48.61 25.535) (end 46.875 23.8) (width 0.508) (layer "B.Cu") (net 6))
 (segment (start 62.804999 24.265) (end 63.57 25.030001) (width 0.508) (layer "B.Cu") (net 3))
 (segment (start 55.4 24.265) (end 62.804999 24.265) (width 0.508) (layer "B.Cu") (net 3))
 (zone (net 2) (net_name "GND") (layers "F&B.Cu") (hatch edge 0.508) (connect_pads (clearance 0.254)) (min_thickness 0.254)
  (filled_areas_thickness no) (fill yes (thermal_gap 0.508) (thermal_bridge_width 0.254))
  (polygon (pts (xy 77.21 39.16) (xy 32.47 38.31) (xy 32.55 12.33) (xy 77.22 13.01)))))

